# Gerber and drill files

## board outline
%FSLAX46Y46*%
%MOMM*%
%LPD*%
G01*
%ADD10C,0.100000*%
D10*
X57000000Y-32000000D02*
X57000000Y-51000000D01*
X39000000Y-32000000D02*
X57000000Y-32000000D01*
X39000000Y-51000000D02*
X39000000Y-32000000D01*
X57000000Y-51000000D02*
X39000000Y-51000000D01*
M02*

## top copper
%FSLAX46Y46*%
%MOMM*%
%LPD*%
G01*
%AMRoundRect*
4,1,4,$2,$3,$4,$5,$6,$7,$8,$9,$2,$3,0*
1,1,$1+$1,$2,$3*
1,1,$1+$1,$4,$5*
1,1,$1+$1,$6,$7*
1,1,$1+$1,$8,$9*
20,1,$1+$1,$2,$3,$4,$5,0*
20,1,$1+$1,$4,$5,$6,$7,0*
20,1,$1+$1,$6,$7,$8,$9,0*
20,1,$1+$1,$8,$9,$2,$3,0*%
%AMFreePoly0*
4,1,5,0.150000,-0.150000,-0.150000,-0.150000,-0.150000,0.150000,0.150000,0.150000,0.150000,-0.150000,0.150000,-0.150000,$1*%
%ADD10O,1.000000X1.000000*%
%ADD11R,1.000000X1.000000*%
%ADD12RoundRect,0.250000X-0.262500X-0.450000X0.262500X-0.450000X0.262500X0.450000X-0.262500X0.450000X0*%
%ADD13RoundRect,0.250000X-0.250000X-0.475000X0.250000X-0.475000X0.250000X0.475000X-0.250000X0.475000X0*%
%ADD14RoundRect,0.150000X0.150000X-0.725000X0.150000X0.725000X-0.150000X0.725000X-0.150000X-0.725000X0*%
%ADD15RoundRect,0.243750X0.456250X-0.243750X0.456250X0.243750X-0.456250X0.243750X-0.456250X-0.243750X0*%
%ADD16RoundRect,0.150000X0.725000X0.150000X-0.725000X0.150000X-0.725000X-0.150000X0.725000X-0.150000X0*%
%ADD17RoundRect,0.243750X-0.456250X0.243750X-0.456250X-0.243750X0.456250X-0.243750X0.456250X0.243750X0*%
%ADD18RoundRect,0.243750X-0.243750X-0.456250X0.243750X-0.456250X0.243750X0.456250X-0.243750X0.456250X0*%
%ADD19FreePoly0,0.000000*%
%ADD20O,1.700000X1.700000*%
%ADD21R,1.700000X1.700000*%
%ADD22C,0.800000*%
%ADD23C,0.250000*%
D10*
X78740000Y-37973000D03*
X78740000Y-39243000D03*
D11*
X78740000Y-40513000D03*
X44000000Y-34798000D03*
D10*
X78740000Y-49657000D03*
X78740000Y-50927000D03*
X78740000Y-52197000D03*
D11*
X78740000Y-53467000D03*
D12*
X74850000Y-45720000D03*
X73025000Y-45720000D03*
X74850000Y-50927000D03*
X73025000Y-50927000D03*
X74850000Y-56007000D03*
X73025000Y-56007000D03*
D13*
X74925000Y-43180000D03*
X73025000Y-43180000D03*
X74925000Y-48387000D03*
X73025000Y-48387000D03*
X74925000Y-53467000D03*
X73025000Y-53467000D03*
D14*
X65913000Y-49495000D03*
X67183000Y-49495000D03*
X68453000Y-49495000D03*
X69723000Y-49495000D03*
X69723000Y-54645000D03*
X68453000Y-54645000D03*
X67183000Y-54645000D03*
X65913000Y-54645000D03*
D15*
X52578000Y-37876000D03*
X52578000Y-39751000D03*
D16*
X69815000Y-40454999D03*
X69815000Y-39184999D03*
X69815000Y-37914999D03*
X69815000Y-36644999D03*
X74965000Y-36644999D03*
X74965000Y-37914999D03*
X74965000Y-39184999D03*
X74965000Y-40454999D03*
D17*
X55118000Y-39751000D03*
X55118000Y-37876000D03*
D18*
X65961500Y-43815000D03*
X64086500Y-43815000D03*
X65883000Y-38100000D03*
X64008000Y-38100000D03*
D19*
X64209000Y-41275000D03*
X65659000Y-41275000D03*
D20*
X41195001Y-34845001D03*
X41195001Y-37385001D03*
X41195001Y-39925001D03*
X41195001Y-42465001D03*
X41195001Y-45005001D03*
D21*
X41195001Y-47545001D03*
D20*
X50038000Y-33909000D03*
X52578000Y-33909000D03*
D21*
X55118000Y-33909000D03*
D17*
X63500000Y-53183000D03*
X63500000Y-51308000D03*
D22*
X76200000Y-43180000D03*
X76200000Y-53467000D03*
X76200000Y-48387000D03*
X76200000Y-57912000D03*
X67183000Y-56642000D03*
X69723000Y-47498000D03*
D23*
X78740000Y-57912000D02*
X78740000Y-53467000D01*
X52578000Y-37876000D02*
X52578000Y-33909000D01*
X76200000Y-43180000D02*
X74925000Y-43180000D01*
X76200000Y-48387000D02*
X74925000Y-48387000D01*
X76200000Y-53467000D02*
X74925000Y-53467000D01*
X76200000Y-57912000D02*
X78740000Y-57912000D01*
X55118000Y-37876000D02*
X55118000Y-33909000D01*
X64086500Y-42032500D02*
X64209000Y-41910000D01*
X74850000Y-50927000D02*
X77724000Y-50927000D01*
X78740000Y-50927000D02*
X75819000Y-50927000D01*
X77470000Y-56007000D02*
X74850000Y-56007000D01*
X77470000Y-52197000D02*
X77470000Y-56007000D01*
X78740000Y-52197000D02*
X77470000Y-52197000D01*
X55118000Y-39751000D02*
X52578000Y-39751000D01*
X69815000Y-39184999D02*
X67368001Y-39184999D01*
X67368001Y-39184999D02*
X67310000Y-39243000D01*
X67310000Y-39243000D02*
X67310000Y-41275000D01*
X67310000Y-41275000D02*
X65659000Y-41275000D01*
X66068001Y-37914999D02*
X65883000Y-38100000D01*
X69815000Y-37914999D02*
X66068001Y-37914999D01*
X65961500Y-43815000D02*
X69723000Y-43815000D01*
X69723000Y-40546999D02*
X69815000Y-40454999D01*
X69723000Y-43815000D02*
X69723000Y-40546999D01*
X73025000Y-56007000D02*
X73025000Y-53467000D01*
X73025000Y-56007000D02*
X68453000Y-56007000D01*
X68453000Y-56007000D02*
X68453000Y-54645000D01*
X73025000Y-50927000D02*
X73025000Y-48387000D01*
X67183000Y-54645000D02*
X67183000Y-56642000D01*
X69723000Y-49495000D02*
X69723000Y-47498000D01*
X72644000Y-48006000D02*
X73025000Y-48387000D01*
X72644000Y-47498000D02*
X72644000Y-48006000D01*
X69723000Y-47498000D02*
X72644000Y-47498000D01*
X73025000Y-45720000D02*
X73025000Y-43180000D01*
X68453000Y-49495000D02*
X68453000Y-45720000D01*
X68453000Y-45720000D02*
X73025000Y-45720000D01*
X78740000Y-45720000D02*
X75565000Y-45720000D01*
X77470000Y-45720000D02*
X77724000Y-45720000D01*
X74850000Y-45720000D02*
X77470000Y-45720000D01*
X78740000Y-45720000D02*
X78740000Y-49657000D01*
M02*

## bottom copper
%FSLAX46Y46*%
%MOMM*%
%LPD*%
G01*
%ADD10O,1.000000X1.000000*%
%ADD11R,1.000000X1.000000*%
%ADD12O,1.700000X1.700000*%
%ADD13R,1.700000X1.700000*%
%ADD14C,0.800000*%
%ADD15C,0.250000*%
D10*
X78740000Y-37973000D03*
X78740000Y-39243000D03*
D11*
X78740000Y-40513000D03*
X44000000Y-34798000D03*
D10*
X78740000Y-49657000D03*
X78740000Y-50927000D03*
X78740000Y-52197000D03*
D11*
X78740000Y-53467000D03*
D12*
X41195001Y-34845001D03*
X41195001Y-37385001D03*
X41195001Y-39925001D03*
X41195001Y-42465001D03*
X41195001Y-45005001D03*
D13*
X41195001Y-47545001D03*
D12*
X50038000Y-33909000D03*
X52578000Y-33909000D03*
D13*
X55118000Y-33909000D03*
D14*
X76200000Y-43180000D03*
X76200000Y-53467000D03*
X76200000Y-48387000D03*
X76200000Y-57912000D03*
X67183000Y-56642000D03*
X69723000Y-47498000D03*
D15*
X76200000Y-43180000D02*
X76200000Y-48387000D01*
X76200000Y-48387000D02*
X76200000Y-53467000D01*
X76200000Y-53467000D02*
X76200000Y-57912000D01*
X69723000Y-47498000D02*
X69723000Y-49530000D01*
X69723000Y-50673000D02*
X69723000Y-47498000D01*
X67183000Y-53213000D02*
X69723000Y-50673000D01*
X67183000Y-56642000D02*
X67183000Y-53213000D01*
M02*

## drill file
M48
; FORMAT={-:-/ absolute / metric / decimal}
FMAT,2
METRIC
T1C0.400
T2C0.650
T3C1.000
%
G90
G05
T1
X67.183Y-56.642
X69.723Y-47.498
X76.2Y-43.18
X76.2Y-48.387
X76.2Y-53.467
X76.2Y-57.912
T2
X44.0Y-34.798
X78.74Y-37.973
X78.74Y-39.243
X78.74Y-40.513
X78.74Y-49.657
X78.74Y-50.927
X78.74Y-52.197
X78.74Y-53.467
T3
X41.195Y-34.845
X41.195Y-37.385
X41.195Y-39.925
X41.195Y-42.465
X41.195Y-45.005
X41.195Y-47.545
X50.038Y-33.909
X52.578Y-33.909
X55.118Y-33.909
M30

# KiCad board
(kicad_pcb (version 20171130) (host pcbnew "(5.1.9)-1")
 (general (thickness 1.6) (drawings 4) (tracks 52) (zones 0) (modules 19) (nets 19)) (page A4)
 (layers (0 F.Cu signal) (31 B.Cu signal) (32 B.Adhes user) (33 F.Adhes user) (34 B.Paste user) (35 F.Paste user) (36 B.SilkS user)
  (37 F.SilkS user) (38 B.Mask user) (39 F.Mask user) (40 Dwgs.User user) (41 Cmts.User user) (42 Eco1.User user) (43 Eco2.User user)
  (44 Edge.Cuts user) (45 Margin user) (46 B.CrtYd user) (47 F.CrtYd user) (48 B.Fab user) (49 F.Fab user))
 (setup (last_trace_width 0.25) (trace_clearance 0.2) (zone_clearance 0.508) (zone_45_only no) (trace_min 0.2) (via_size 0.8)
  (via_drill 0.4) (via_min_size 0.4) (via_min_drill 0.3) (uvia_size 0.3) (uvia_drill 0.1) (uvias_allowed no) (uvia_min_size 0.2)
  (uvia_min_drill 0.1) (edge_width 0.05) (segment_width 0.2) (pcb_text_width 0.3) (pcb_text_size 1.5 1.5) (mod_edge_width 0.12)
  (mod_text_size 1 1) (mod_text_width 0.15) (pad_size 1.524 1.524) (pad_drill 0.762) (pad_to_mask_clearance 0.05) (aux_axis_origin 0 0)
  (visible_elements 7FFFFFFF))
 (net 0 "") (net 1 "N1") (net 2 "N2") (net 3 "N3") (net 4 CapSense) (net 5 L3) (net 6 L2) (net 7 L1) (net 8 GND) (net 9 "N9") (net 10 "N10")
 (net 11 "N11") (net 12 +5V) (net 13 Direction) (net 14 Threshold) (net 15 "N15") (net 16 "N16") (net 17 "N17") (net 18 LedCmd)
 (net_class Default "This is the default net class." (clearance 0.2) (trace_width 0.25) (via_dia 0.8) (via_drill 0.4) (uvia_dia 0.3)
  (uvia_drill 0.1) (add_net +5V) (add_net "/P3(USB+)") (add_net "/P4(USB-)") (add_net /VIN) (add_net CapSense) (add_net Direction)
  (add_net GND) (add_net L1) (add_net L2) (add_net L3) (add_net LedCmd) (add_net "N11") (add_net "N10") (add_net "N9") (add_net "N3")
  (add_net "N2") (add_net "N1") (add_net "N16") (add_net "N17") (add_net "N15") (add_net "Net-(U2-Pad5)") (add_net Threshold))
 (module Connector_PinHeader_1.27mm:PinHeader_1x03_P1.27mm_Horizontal (layer B.Cu) (at 78.74 40.513)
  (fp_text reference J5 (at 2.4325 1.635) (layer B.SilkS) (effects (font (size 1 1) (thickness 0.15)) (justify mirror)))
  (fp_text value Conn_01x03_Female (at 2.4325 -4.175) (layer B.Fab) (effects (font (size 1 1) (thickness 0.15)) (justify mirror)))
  (pad 3 thru_hole oval (at 0 -2.54) (size 1 1) (drill 0.65) (layers *.Cu *.Mask) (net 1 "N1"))
  (pad 2 thru_hole oval (at 0 -1.27) (size 1 1) (drill 0.65) (layers *.Cu *.Mask) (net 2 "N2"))
  (pad 1 thru_hole rect (at 0 0) (size 1 1) (drill 0.65) (layers *.Cu *.Mask) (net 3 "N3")))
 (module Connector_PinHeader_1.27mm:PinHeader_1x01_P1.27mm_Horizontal (layer B.Cu) (at 44 34.798 90)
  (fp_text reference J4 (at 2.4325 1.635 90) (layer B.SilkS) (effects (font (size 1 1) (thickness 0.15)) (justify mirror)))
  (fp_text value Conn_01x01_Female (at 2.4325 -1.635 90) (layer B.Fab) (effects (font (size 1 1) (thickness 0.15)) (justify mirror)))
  (pad 1 thru_hole rect (at 0 0 90) (size 1 1) (drill 0.65) (layers *.Cu *.Mask) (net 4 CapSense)))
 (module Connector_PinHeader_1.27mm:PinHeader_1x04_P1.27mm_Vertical (layer B.Cu) (at 78.74 53.467)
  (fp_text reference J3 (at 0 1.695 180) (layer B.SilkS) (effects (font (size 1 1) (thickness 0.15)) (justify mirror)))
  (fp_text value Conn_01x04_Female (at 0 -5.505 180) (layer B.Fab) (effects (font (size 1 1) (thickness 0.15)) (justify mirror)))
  (pad 4 thru_hole oval (at 0 -3.81) (size 1 1) (drill 0.65) (layers *.Cu *.Mask) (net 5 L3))
  (pad 3 thru_hole oval (at 0 -2.54) (size 1 1) (drill 0.65) (layers *.Cu *.Mask) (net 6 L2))
  (pad 2 thru_hole oval (at 0 -1.27) (size 1 1) (drill 0.65) (layers *.Cu *.Mask) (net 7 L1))
  (pad 1 thru_hole rect (at 0 0) (size 1 1) (drill 0.65) (layers *.Cu *.Mask) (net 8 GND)))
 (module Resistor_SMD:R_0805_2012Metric (layer F.Cu) (at 73.9375 45.72)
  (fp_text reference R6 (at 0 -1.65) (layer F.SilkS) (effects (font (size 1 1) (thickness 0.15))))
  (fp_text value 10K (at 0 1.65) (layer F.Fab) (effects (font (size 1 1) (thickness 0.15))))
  (pad 2 smd roundrect (at 0.9125 0) (size 1.025 1.4) (layers F.Cu F.Paste F.Mask) (roundrect_rratio 0.243902) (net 5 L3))
  (pad 1 smd roundrect (at -0.9125 0) (size 1.025 1.4) (layers F.Cu F.Paste F.Mask) (roundrect_rratio 0.243902) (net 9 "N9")))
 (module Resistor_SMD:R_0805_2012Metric (layer F.Cu) (at 73.9375 50.927)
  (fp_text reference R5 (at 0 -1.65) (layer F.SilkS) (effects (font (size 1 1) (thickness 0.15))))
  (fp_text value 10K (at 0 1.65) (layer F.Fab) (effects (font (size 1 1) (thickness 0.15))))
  (pad 2 smd roundrect (at 0.9125 0) (size 1.025 1.4) (layers F.Cu F.Paste F.Mask) (roundrect_rratio 0.243902) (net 6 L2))
  (pad 1 smd roundrect (at -0.9125 0) (size 1.025 1.4) (layers F.Cu F.Paste F.Mask) (roundrect_rratio 0.243902) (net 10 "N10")))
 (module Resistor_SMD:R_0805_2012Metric (layer F.Cu) (at 73.9375 56.007)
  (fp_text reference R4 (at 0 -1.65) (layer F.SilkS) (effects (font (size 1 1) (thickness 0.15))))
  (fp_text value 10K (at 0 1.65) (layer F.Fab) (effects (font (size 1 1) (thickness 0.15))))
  (pad 2 smd roundrect (at 0.9125 0) (size 1.025 1.4) (layers F.Cu F.Paste F.Mask) (roundrect_rratio 0.243902) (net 7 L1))
  (pad 1 smd roundrect (at -0.9125 0) (size 1.025 1.4) (layers F.Cu F.Paste F.Mask) (roundrect_rratio 0.243902) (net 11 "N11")))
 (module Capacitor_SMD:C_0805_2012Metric (layer F.Cu) (at 73.975 43.18)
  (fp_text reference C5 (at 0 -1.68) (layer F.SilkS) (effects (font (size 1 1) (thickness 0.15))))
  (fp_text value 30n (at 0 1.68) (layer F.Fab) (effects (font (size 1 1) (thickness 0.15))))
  (pad 2 smd roundrect (at 0.95 0) (size 1 1.45) (layers F.Cu F.Paste F.Mask) (roundrect_rratio 0.25) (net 8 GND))
  (pad 1 smd roundrect (at -0.95 0) (size 1 1.45) (layers F.Cu F.Paste F.Mask) (roundrect_rratio 0.25) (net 9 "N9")))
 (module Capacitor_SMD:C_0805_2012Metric (layer F.Cu) (at 73.975 48.387)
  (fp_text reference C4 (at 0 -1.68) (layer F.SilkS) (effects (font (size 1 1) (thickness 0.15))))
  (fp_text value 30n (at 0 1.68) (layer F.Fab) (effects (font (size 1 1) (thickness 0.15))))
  (pad 2 smd roundrect (at 0.95 0) (size 1 1.45) (layers F.Cu F.Paste F.Mask) (roundrect_rratio 0.25) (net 8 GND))
  (pad 1 smd roundrect (at -0.95 0) (size 1 1.45) (layers F.Cu F.Paste F.Mask) (roundrect_rratio 0.25) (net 10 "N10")))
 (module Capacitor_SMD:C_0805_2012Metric (layer F.Cu) (at 73.975 53.467)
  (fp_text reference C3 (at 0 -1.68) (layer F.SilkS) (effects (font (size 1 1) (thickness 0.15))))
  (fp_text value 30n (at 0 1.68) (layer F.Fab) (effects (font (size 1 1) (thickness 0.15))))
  (pad 2 smd roundrect (at 0.95 0) (size 1 1.45) (layers F.Cu F.Paste F.Mask) (roundrect_rratio 0.25) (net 8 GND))
  (pad 1 smd roundrect (at -0.95 0) (size 1 1.45) (layers F.Cu F.Paste F.Mask) (roundrect_rratio 0.25) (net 11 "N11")))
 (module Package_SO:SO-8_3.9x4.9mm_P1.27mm (layer F.Cu) (at 67.818 52.07 90)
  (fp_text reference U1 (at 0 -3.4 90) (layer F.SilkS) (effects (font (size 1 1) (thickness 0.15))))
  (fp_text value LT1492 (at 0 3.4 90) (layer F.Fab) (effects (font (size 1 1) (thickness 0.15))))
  (pad 8 smd roundrect (at 2.575 -1.905 90) (size 1.75 0.6) (layers F.Cu F.Paste F.Mask) (roundrect_rratio 0.25) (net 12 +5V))
  (pad 7 smd roundrect (at 2.575 -0.635 90) (size 1.75 0.6) (layers F.Cu F.Paste F.Mask) (roundrect_rratio 0.25) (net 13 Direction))
  (pad 6 smd roundrect (at 2.575 0.635 90) (size 1.75 0.6) (layers F.Cu F.Paste F.Mask) (roundrect_rratio 0.25) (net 9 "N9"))
  (pad 5 smd roundrect (at 2.575 1.905 90) (size 1.75 0.6) (layers F.Cu F.Paste F.Mask) (roundrect_rratio 0.25) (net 10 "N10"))
  (pad 4 smd roundrect (at -2.575 1.905 90) (size 1.75 0.6) (layers F.Cu F.Paste F.Mask) (roundrect_rratio 0.25) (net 8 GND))
  (pad 3 smd roundrect (at -2.575 0.635 90) (size 1.75 0.6) (layers F.Cu F.Paste F.Mask) (roundrect_rratio 0.25) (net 11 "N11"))
  (pad 2 smd roundrect (at -2.575 -0.635 90) (size 1.75 0.6) (layers F.Cu F.Paste F.Mask) (roundrect_rratio 0.25) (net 10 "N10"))
  (pad 1 smd roundrect (at -2.575 -1.905 90) (size 1.75 0.6) (layers F.Cu F.Paste F.Mask) (roundrect_rratio 0.25) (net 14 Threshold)))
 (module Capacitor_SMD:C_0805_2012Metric (layer F.Cu) (at 52.578 38.8135 90)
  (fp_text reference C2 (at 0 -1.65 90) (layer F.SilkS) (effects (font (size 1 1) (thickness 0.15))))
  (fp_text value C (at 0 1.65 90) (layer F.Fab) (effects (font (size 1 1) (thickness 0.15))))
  (pad 2 smd roundrect (at 0.9375 0 90) (size 0.975 1.4) (layers F.Cu F.Paste F.Mask) (roundrect_rratio 0.25) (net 8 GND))
  (pad 1 smd roundrect (at -0.9375 0 90) (size 0.975 1.4) (layers F.Cu F.Paste F.Mask) (roundrect_rratio 0.25) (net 4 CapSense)))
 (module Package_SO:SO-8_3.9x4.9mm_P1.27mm (layer F.Cu) (at 72.39 38.549999 180)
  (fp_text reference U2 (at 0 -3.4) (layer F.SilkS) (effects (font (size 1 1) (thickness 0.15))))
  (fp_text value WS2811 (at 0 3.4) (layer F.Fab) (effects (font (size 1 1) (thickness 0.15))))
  (pad 8 smd roundrect (at 2.575 -1.905 180) (size 1.75 0.6) (layers F.Cu F.Paste F.Mask) (roundrect_rratio 0.25) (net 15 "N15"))
  (pad 7 smd roundrect (at 2.575 -0.635 180) (size 1.75 0.6) (layers F.Cu F.Paste F.Mask) (roundrect_rratio 0.25) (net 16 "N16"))
  (pad 6 smd roundrect (at 2.575 0.635 180) (size 1.75 0.6) (layers F.Cu F.Paste F.Mask) (roundrect_rratio 0.25) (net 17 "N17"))
  (pad 5 smd roundrect (at 2.575 1.905 180) (size 1.75 0.6) (layers F.Cu F.Paste F.Mask) (roundrect_rratio 0.25))
  (pad 4 smd roundrect (at -2.575 1.905 180) (size 1.75 0.6) (layers F.Cu F.Paste F.Mask) (roundrect_rratio 0.25) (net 8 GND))
  (pad 3 smd roundrect (at -2.575 0.635 180) (size 1.75 0.6) (layers F.Cu F.Paste F.Mask) (roundrect_rratio 0.25) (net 1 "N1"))
  (pad 2 smd roundrect (at -2.575 -0.635 180) (size 1.75 0.6) (layers F.Cu F.Paste F.Mask) (roundrect_rratio 0.25) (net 2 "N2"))
  (pad 1 smd roundrect (at -2.575 -1.905 180) (size 1.75 0.6) (layers F.Cu F.Paste F.Mask) (roundrect_rratio 0.25) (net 3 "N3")))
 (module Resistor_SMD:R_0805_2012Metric (layer F.Cu) (at 55.118 38.8135 270)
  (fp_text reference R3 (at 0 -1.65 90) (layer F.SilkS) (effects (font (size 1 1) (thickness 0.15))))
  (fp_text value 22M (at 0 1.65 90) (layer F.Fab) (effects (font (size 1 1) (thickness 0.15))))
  (pad 2 smd roundrect (at 0.9375 0 270) (size 0.975 1.4) (layers F.Cu F.Paste F.Mask) (roundrect_rratio 0.25) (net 4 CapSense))
  (pad 1 smd roundrect (at -0.9375 0 270) (size 0.975 1.4) (layers F.Cu F.Paste F.Mask) (roundrect_rratio 0.25) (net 12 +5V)))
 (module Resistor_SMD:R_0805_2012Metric (layer F.Cu) (at 65.024 43.815)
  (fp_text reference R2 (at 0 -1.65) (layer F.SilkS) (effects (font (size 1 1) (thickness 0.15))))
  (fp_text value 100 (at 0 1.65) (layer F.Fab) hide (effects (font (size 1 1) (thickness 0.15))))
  (pad 2 smd roundrect (at 0.9375 0) (size 0.975 1.4) (layers F.Cu F.Paste F.Mask) (roundrect_rratio 0.25) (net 15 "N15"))
  (pad 1 smd roundrect (at -0.9375 0) (size 0.975 1.4) (layers F.Cu F.Paste F.Mask) (roundrect_rratio 0.25) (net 12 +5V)))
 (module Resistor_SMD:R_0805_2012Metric (layer F.Cu) (at 64.9455 38.1)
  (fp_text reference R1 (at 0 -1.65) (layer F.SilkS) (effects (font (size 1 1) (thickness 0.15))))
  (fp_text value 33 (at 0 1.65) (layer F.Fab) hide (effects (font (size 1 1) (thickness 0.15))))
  (pad 2 smd roundrect (at 0.9375 0) (size 0.975 1.4) (layers F.Cu F.Paste F.Mask) (roundrect_rratio 0.25) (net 17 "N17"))
  (pad 1 smd roundrect (at -0.9375 0) (size 0.975 1.4) (layers F.Cu F.Paste F.Mask) (roundrect_rratio 0.25) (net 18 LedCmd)))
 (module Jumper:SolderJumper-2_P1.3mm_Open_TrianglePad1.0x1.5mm (layer F.Cu) (at 64.934 41.275)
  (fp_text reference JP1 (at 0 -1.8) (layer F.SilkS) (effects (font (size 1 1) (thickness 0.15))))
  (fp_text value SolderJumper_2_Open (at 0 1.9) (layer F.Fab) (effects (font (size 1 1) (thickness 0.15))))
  (pad 1 smd custom (at -0.725 0) (size 0.3 0.3) (layers F.Cu F.Mask) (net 12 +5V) (zone_connect 2)
   (options (clearance outline) (anchor rect)) (primitives))
  (pad 2 smd custom (at 0.725 0) (size 0.3 0.3) (layers F.Cu F.Mask) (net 16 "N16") (zone_connect 2)
   (options (clearance outline) (anchor rect)) (primitives)))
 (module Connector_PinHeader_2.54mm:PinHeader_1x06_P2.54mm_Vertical (layer B.Cu) (at 41.195001 47.545001)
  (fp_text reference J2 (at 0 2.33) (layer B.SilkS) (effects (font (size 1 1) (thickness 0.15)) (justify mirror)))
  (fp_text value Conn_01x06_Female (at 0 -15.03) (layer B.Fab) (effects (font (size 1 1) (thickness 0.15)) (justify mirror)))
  (pad 6 thru_hole oval (at 0 -12.7) (size 1.7 1.7) (drill 1) (layers *.Cu *.Mask) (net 4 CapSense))
  (pad 5 thru_hole oval (at 0 -10.16) (size 1.7 1.7) (drill 1) (layers *.Cu *.Mask))
  (pad 4 thru_hole oval (at 0 -7.62) (size 1.7 1.7) (drill 1) (layers *.Cu *.Mask))
  (pad 3 thru_hole oval (at 0 -5.08) (size 1.7 1.7) (drill 1) (layers *.Cu *.Mask) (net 14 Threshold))
  (pad 2 thru_hole oval (at 0 -2.54) (size 1.7 1.7) (drill 1) (layers *.Cu *.Mask) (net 13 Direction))
  (pad 1 thru_hole rect (at 0 0) (size 1.7 1.7) (drill 1) (layers *.Cu *.Mask) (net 18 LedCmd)))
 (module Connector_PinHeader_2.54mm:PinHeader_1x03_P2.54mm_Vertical (layer B.Cu) (at 55.118 33.909 90)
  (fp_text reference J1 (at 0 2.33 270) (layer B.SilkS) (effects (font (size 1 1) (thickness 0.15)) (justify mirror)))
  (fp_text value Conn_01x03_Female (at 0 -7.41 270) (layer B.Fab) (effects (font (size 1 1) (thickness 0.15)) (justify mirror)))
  (pad 3 thru_hole oval (at 0 -5.08 90) (size 1.7 1.7) (drill 1) (layers *.Cu *.Mask))
  (pad 2 thru_hole oval (at 0 -2.54 90) (size 1.7 1.7) (drill 1) (layers *.Cu *.Mask) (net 8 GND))
  (pad 1 thru_hole rect (at 0 0 90) (size 1.7 1.7) (drill 1) (layers *.Cu *.Mask) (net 12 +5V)))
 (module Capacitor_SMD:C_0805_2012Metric (layer F.Cu) (at 63.5 52.2455 270)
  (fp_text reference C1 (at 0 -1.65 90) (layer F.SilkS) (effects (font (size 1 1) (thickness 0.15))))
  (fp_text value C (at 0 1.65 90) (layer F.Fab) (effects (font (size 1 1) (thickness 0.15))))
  (pad 2 smd roundrect (at 0.9375 0 270) (size 0.975 1.4) (layers F.Cu F.Paste F.Mask) (roundrect_rratio 0.25) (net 8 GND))
  (pad 1 smd roundrect (at -0.9375 0 270) (size 0.975 1.4) (layers F.Cu F.Paste F.Mask) (roundrect_rratio 0.25) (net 12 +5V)))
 (gr_line (start 57 32) (end 57 51) (layer Edge.Cuts) (width 0.1))
 (gr_line (start 39 32) (end 57 32) (layer Edge.Cuts) (width 0.1))
 (gr_line (start 39 51) (end 39 32) (layer Edge.Cuts) (width 0.1))
 (gr_line (start 57 51) (end 39 51) (layer Edge.Cuts) (width 0.1))
 (via (at 76.2 43.18) (size 0.8) (drill 0.4) (layers F.Cu B.Cu) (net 8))
 (segment (start 76.2 43.18) (end 76.2 48.387) (width 0.25) (layer B.Cu) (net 8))
 (via (at 76.2 53.467) (size 0.8) (drill 0.4) (layers F.Cu B.Cu) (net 8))
 (segment (start 76.2 48.387) (end 76.2 53.467) (width 0.25) (layer B.Cu) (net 8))
 (via (at 76.2 48.387) (size 0.8) (drill 0.4) (layers F.Cu B.Cu) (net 8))
 (via (at 76.2 57.912) (size 0.8) (drill 0.4) (layers F.Cu B.Cu) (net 8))
 (segment (start 76.2 53.467) (end 76.2 57.912) (width 0.25) (layer B.Cu) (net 8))
 (segment (start 78.74 57.912) (end 78.74 53.467) (width 0.25) (layer F.Cu) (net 8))
 (segment (start 52.578 37.876) (end 52.578 33.909) (width 0.25) (layer F.Cu) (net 8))
 (segment (start 76.2 43.18) (end 74.925 43.18) (width 0.25) (layer F.Cu) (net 8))
 (segment (start 76.2 48.387) (end 74.925 48.387) (width 0.25) (layer F.Cu) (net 8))
 (segment (start 76.2 53.467) (end 74.925 53.467) (width 0.25) (layer F.Cu) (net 8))
 (segment (start 76.2 57.912) (end 78.74 57.912) (width 0.25) (layer F.Cu) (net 8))
 (segment (start 55.118 37.876) (end 55.118 33.909) (width 0.25) (layer F.Cu) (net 12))
 (segment (start 64.0865 42.0325) (end 64.209 41.91) (width 0.25) (layer F.Cu) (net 12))
 (segment (start 74.85 50.927) (end 77.724 50.927) (width 0.25) (layer F.Cu) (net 6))
 (segment (start 78.74 50.927) (end 75.819 50.927) (width 0.25) (layer F.Cu) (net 6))
 (segment (start 77.47 56.007) (end 74.85 56.007) (width 0.25) (layer F.Cu) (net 7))
 (segment (start 77.47 52.197) (end 77.47 56.007) (width 0.25) (layer F.Cu) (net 7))
 (segment (start 78.74 52.197) (end 77.47 52.197) (width 0.25) (layer F.Cu) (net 7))
 (segment (start 55.118 39.751) (end 52.578 39.751) (width 0.25) (layer F.Cu) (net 4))
 (segment (start 69.815 39.184999) (end 67.368001 39.184999) (width 0.25) (layer F.Cu) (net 16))
 (segment (start 67.368001 39.184999) (end 67.31 39.243) (width 0.25) (layer F.Cu) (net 16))
 (segment (start 67.31 39.243) (end 67.31 41.275) (width 0.25) (layer F.Cu) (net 16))
 (segment (start 67.31 41.275) (end 65.659 41.275) (width 0.25) (layer F.Cu) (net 16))
 (segment (start 66.068001 37.914999) (end 65.883 38.1) (width 0.25) (layer F.Cu) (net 17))
 (segment (start 69.815 37.914999) (end 66.068001 37.914999) (width 0.25) (layer F.Cu) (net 17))
 (segment (start 65.9615 43.815) (end 69.723 43.815) (width 0.25) (layer F.Cu) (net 15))
 (segment (start 69.723 40.546999) (end 69.815 40.454999) (width 0.25) (layer F.Cu) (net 15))
 (segment (start 69.723 43.815) (end 69.723 40.546999) (width 0.25) (layer F.Cu) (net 15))
 (segment (start 73.025 56.007) (end 73.025 53.467) (width 0.25) (layer F.Cu) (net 11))
 (segment (start 73.025 56.007) (end 68.453 56.007) (width 0.25) (layer F.Cu) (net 11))
 (segment (start 68.453 56.007) (end 68.453 54.645) (width 0.25) (layer F.Cu) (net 11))
 (segment (start 73.025 50.927) (end 73.025 48.387) (width 0.25) (layer F.Cu) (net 10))
 (segment (start 67.183 54.645) (end 67.183 56.642) (width 0.25) (layer F.Cu) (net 10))
 (via (at 67.183 56.642) (size 0.8) (drill 0.4) (layers F.Cu B.Cu) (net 10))
 (via (at 69.723 47.498) (size 0.8) (drill 0.4) (layers F.Cu B.Cu) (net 10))
 (segment (start 69.723 49.495) (end 69.723 47.498) (width 0.25) (layer F.Cu) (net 10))
 (segment (start 69.723 47.498) (end 69.723 49.53) (width 0.25) (layer B.Cu) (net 10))
 (segment (start 69.723 50.673) (end 69.723 47.498) (width 0.25) (layer B.Cu) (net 10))
 (segment (start 67.183 53.213) (end 69.723 50.673) (width 0.25) (layer B.Cu) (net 10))
 (segment (start 67.183 56.642) (end 67.183 53.213) (width 0.25) (layer B.Cu) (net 10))
 (segment (start 72.644 48.006) (end 73.025 48.387) (width 0.25) (layer F.Cu) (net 10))
 (segment (start 72.644 47.498) (end 72.644 48.006) (width 0.25) (layer F.Cu) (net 10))
 (segment (start 69.723 47.498) (end 72.644 47.498) (width 0.25) (layer F.Cu) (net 10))
 (segment (start 73.025 45.72) (end 73.025 43.18) (width 0.25) (layer F.Cu) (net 9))
 (segment (start 68.453 49.495) (end 68.453 45.72) (width 0.25) (layer F.Cu) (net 9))
 (segment (start 68.453 45.72) (end 73.025 45.72) (width 0.25) (layer F.Cu) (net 9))
 (segment (start 78.74 45.72) (end 75.565 45.72) (width 0.25) (layer F.Cu) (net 5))
 (segment (start 77.47 45.72) (end 77.724 45.72) (width 0.25) (layer F.Cu) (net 5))
 (segment (start 74.85 45.72) (end 77.47 45.72) (width 0.25) (layer F.Cu) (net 5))
 (segment (start 78.74 45.72) (end 78.74 49.657) (width 0.25) (layer F.Cu) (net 5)))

